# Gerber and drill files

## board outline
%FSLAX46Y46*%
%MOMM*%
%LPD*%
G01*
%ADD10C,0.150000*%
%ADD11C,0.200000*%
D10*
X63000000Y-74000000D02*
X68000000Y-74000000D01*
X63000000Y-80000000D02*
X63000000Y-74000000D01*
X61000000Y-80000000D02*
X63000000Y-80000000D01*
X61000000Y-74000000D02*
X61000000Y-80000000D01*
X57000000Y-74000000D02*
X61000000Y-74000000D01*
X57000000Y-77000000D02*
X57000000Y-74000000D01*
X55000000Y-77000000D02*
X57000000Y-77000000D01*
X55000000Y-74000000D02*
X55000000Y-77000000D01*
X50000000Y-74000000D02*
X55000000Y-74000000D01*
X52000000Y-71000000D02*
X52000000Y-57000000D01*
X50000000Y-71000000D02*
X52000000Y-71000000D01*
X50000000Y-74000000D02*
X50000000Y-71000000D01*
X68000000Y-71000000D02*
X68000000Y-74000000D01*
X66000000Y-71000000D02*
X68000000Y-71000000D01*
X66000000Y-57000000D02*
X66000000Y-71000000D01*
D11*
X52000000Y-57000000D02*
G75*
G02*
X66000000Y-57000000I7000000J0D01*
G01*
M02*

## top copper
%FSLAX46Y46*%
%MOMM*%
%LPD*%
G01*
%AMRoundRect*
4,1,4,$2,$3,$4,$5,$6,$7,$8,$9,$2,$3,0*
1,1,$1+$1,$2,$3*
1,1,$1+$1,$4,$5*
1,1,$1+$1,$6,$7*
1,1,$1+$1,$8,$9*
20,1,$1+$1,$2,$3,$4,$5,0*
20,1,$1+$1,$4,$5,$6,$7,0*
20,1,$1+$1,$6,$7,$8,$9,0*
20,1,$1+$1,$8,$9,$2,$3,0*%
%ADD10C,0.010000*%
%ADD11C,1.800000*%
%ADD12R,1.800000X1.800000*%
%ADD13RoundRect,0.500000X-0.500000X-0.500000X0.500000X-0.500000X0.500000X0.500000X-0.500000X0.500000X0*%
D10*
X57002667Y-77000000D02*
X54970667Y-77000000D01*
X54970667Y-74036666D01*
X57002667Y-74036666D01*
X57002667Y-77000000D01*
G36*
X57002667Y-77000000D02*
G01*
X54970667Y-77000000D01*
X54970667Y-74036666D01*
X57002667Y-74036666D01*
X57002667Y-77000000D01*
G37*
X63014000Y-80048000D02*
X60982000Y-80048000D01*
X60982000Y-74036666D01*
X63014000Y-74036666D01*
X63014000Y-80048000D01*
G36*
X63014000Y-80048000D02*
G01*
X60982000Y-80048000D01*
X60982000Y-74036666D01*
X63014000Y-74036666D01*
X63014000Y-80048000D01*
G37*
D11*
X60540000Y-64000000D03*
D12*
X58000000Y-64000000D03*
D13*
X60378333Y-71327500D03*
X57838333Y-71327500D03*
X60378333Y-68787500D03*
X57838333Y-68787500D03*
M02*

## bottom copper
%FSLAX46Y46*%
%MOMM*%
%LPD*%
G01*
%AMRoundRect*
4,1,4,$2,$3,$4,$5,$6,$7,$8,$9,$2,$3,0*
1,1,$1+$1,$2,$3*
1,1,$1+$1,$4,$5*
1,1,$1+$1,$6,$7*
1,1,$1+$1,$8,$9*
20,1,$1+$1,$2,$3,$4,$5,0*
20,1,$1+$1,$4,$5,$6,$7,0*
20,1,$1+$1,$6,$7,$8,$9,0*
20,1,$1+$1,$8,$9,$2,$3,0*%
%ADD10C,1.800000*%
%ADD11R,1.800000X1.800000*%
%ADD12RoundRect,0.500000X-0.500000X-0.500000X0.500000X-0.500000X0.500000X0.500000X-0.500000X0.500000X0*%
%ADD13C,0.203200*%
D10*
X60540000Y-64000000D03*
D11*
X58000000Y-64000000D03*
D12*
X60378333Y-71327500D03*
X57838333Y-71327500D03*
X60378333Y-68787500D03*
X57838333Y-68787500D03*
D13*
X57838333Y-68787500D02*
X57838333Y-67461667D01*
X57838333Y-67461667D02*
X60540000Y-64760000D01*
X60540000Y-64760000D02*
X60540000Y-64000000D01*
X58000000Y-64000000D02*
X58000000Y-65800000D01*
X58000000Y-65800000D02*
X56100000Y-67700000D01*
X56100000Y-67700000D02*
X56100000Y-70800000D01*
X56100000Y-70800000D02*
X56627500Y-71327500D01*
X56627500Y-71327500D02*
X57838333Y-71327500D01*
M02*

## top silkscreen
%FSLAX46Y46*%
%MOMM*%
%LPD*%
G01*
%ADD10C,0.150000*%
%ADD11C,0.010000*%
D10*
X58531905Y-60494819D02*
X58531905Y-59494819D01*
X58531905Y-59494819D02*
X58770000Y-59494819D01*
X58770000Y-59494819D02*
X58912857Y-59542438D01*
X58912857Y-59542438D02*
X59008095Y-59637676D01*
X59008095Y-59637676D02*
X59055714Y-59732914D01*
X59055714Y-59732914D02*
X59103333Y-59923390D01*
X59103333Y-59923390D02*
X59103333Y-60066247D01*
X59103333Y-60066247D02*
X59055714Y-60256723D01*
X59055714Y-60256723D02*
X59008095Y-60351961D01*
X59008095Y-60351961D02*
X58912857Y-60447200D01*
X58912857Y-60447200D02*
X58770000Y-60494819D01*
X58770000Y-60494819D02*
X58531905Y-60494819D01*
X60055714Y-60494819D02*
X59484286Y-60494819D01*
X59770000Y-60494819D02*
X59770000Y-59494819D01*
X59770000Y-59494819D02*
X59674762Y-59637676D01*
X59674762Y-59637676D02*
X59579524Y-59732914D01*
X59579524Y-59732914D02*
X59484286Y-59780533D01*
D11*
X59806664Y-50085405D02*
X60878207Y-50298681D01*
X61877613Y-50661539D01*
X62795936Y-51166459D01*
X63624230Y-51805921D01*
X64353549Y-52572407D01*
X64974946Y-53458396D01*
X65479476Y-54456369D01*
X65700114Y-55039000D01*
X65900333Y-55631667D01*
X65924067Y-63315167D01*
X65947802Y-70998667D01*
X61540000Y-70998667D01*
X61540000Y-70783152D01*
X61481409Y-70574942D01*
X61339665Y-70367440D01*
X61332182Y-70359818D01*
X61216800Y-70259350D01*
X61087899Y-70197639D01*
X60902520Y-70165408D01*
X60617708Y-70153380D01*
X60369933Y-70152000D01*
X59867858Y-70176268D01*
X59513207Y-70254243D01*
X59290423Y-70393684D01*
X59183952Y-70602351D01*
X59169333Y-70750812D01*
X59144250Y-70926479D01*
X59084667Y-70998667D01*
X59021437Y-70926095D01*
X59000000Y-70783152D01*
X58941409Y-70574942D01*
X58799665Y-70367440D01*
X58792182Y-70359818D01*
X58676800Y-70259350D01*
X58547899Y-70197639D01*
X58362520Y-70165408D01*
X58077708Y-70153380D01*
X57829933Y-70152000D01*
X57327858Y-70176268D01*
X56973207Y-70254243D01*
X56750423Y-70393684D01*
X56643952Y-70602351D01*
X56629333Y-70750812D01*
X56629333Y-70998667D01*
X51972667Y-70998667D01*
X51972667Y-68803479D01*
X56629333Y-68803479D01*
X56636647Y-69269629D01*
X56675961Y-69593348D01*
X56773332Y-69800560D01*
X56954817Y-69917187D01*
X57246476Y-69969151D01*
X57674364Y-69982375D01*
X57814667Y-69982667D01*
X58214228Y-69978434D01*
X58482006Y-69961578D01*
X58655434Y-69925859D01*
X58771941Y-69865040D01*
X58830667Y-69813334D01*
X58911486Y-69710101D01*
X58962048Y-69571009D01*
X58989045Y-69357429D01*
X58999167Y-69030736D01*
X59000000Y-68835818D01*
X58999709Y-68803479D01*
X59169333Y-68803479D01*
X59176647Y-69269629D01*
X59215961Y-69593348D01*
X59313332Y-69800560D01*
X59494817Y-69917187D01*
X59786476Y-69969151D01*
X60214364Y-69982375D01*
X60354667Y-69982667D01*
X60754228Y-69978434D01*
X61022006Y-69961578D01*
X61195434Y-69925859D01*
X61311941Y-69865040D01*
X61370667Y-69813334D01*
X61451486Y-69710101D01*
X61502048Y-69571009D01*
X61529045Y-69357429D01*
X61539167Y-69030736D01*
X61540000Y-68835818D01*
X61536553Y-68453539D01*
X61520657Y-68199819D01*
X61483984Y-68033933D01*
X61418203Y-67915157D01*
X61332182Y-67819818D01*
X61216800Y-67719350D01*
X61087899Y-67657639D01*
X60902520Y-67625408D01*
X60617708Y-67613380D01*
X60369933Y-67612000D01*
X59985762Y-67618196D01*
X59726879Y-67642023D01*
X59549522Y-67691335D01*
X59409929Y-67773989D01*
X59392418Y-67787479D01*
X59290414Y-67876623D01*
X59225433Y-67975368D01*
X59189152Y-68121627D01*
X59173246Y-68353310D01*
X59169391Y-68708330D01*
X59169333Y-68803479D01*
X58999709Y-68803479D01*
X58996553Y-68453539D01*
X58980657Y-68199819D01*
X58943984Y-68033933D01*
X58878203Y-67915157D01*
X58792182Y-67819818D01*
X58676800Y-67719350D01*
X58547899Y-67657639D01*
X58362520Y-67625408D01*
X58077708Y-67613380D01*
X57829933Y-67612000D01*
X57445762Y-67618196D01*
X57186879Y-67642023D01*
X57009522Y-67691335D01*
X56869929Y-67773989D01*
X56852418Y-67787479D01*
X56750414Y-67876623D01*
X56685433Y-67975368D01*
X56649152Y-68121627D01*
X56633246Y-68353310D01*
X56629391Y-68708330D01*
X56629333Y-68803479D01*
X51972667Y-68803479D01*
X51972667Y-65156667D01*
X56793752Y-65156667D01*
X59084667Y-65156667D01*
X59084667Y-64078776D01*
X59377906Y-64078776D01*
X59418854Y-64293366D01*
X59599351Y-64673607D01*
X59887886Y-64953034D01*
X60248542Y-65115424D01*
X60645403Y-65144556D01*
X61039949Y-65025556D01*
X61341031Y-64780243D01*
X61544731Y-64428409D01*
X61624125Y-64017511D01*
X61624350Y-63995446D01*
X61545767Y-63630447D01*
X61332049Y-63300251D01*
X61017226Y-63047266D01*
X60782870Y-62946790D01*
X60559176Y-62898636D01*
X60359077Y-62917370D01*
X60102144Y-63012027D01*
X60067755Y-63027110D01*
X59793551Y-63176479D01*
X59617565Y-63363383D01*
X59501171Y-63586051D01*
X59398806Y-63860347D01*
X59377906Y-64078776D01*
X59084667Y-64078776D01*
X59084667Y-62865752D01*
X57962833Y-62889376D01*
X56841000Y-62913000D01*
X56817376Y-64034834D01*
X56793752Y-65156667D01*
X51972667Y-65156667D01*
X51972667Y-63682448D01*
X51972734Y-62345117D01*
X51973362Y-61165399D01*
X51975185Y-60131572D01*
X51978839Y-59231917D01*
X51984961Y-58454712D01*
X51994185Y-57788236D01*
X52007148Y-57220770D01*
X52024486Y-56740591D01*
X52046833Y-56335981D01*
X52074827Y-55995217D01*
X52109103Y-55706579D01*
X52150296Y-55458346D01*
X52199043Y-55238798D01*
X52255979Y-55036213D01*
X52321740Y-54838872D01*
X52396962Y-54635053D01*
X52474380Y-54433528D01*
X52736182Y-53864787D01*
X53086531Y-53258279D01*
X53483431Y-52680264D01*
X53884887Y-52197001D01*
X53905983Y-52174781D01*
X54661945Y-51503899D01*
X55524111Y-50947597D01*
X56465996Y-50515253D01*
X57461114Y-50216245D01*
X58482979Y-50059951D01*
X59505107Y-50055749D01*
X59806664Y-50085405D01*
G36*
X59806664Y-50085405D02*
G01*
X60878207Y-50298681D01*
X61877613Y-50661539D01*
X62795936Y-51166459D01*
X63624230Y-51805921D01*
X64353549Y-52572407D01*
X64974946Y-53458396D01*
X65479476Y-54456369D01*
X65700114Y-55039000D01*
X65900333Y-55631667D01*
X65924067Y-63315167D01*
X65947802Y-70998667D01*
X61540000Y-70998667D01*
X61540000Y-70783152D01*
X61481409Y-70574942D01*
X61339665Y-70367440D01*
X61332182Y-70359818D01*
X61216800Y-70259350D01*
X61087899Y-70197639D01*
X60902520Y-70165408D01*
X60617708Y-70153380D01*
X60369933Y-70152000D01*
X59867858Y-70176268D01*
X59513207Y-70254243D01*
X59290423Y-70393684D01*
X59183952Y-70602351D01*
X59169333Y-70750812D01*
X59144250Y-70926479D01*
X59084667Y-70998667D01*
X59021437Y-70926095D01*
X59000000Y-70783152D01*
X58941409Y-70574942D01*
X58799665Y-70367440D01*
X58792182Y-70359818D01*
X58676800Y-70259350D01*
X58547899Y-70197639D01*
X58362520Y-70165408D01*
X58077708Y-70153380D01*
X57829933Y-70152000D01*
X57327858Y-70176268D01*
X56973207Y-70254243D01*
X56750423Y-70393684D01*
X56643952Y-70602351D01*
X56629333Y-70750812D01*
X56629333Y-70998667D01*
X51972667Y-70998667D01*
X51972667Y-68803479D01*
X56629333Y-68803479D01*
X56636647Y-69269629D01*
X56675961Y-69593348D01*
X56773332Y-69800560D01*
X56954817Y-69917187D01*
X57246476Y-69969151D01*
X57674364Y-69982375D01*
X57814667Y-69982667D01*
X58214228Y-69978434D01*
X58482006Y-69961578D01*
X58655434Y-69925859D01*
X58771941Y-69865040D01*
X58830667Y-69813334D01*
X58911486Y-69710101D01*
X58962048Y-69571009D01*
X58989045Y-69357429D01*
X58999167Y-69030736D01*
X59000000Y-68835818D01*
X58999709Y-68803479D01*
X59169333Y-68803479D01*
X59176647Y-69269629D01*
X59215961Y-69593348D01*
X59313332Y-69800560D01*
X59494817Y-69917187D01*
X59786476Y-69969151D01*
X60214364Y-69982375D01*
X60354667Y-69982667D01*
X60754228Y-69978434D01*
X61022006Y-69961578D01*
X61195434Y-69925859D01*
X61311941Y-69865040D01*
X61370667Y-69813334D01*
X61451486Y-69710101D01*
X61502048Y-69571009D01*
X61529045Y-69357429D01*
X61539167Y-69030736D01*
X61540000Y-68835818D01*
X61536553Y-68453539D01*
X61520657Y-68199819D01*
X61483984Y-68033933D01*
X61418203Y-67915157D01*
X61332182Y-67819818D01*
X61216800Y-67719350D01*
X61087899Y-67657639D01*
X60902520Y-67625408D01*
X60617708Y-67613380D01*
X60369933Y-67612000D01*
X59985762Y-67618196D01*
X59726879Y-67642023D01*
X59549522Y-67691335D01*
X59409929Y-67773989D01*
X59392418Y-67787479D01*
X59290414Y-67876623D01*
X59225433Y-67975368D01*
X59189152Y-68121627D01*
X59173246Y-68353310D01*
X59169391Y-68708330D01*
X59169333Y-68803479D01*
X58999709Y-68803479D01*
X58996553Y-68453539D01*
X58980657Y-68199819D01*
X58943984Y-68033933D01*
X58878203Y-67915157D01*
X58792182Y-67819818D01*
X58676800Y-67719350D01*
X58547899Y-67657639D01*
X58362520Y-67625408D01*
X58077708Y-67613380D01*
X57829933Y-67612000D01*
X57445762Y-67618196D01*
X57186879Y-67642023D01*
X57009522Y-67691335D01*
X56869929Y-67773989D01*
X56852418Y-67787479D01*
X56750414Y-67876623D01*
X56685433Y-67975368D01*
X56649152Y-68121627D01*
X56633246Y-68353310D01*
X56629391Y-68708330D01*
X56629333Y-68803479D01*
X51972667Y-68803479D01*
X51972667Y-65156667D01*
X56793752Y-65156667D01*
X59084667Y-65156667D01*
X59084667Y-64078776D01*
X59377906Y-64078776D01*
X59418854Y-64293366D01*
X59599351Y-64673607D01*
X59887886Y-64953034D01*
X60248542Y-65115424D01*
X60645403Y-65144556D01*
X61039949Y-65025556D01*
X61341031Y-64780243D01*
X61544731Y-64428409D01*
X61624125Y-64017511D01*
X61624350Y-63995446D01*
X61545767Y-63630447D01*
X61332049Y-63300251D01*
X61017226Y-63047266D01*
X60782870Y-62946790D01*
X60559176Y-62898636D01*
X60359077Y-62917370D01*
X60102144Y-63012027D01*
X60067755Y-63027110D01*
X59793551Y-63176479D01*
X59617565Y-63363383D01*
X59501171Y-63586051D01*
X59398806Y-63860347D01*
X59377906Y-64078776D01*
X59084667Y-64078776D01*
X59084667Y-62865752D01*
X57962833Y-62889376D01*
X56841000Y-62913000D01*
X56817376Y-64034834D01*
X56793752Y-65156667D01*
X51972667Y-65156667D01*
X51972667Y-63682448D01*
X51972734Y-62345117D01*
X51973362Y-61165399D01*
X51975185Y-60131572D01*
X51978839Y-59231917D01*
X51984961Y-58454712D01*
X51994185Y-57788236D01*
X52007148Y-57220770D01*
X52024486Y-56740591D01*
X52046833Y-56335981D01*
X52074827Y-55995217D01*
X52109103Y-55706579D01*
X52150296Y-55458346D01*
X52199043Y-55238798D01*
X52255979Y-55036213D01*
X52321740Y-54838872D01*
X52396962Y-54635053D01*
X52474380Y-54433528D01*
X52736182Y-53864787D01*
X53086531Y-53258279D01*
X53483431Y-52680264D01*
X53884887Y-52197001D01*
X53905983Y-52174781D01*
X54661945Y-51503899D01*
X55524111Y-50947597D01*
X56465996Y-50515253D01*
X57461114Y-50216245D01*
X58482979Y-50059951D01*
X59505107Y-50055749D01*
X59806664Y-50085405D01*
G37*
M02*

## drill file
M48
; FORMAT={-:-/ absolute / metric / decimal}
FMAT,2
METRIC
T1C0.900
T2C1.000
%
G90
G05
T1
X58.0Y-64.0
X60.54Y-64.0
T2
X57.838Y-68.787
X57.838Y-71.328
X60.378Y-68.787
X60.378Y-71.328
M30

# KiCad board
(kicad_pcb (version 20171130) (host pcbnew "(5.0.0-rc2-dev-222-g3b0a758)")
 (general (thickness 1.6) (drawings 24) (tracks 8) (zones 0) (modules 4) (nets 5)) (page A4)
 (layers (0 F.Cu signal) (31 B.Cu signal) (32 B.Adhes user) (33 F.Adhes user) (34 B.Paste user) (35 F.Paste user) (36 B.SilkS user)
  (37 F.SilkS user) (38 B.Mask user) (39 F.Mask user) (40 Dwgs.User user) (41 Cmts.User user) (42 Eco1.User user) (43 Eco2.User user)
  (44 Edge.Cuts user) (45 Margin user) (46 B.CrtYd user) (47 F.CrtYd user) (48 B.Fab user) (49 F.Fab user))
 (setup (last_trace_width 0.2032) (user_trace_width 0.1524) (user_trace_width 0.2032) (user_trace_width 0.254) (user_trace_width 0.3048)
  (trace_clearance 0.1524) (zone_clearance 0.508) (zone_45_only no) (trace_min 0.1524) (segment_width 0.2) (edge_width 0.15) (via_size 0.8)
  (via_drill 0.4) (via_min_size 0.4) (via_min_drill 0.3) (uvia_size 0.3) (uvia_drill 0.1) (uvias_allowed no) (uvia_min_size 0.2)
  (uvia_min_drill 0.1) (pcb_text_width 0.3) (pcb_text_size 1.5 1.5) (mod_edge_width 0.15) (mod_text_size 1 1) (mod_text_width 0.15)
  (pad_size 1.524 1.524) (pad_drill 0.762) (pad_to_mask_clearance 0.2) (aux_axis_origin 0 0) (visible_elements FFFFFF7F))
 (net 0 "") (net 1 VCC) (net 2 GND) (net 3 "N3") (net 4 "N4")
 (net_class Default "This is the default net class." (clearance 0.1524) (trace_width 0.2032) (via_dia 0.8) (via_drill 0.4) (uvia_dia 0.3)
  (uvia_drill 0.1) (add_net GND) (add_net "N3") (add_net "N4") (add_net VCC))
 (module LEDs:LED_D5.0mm (layer F.Cu) (at 58 64)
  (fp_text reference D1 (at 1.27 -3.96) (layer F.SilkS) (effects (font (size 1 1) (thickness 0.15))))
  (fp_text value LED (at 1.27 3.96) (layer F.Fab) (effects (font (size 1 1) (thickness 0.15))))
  (pad 2 thru_hole circle (at 2.54 0) (size 1.8 1.8) (drill 0.9) (layers *.Cu *.Mask) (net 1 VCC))
  (pad 1 thru_hole rect (at 0 0) (size 1.8 1.8) (drill 0.9) (layers *.Cu *.Mask) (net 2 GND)))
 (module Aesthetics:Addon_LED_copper (layer F.Cu) (at 58.95 77)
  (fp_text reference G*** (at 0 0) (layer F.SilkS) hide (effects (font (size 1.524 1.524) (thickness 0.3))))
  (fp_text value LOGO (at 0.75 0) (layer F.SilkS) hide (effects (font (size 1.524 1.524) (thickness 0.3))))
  (fp_poly
   (pts (xy -1.947333 0) (xy -3.979333 0) (xy -3.979333 -2.963334) (xy -1.947333 -2.963334) (xy -1.947333 0)) (layer F.Cu) (width 0.01))
  (fp_poly (pts (xy 4.064 3.048) (xy 2.032 3.048) (xy 2.032 -2.963334) (xy 4.064 -2.963334) (xy 4.064 3.048)) (layer F.Cu) (width 0.01)))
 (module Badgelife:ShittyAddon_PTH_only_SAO (layer F.Cu) (at 57.838333 68.7875)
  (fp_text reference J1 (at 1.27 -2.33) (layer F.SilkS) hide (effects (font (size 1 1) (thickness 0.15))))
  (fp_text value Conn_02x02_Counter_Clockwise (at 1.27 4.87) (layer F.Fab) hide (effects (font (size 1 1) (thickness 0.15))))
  (pad 3 thru_hole roundrect (at 2.54 2.54) (size 2 2) (drill 1) (layers *.Cu *.Mask) (roundrect_rratio 0.25) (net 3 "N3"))
  (pad 2 thru_hole roundrect (at 0 2.54) (size 2 2) (drill 1) (layers *.Cu *.Mask) (roundrect_rratio 0.25) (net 2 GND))
  (pad 4 thru_hole roundrect (at 2.54 0) (size 2 2) (drill 1) (layers *.Cu *.Mask) (roundrect_rratio 0.25) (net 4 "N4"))
  (pad 1 thru_hole roundrect (at 0 0) (size 2 2) (drill 1) (layers *.Cu *.Mask) (roundrect_rratio 0.25) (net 1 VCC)))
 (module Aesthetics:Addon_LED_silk (layer F.Cu) (at 59 60.5)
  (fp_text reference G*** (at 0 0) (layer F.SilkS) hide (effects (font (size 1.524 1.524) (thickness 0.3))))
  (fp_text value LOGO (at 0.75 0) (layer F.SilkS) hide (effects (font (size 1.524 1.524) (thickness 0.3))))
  (fp_poly
   (pts (xy 0.806664 -10.414595) (xy 1.878207 -10.201319) (xy 2.877613 -9.838461) (xy 3.795936 -9.333541) (xy 4.62423 -8.694079)
    (xy 5.353549 -7.927593) (xy 5.974946 -7.041604) (xy 6.479476 -6.043631) (xy 6.700114 -5.461) (xy 6.900333 -4.868333)
    (xy 6.924067 2.815167) (xy 6.947802 10.498667) (xy 2.54 10.498667) (xy 2.54 10.283152) (xy 2.481409 10.074942) (xy 2.339665 9.86744)
    (xy 2.332182 9.859818) (xy 2.2168 9.75935) (xy 2.087899 9.697639) (xy 1.90252 9.665408) (xy 1.617708 9.65338) (xy 1.369933 9.652)
    (xy 0.867858 9.676268) (xy 0.513207 9.754243) (xy 0.290423 9.893684) (xy 0.183952 10.102351) (xy 0.169333 10.250812)
    (xy 0.14425 10.426479) (xy 0.084667 10.498667) (xy 0.021437 10.426095) (xy 0 10.283152) (xy -0.058591 10.074942) (xy -0.200335 9.86744)
    (xy -0.207818 9.859818) (xy -0.3232 9.75935) (xy -0.452101 9.697639) (xy -0.63748 9.665408) (xy -0.922292 9.65338) (xy -1.170067 9.652)
    (xy -1.672142 9.676268) (xy -2.026793 9.754243) (xy -2.249577 9.893684) (xy -2.356048 10.102351) (xy -2.370667 10.250812)
    (xy -2.370667 10.498667) (xy -7.027333 10.498667) (xy -7.027333 8.303479) (xy -2.370667 8.303479) (xy -2.363353 8.769629)
    (xy -2.324039 9.093348) (xy -2.226668 9.30056) (xy -2.045183 9.417187) (xy -1.753524 9.469151) (xy -1.325636 9.482375)
    (xy -1.185333 9.482667) (xy -0.785772 9.478434) (xy -0.517994 9.461578) (xy -0.344566 9.425859) (xy -0.228059 9.36504)
    (xy -0.169333 9.313334) (xy -0.088514 9.210101) (xy -0.037952 9.071009) (xy -0.010955 8.857429) (xy -0.000833 8.530736) (xy 0 8.335818)
    (xy -0.000291 8.303479) (xy 0.169333 8.303479) (xy 0.176647 8.769629) (xy 0.215961 9.093348) (xy 0.313332 9.30056)
    (xy 0.494817 9.417187) (xy 0.786476 9.469151) (xy 1.214364 9.482375) (xy 1.354667 9.482667) (xy 1.754228 9.478434)
    (xy 2.022006 9.461578) (xy 2.195434 9.425859) (xy 2.311941 9.36504) (xy 2.370667 9.313334) (xy 2.451486 9.210101) (xy 2.502048 9.071009)
    (xy 2.529045 8.857429) (xy 2.539167 8.530736) (xy 2.54 8.335818) (xy 2.536553 7.953539) (xy 2.520657 7.699819) (xy 2.483984 7.533933)
    (xy 2.418203 7.415157) (xy 2.332182 7.319818) (xy 2.2168 7.21935) (xy 2.087899 7.157639) (xy 1.90252 7.125408) (xy 1.617708 7.11338)
    (xy 1.369933 7.112) (xy 0.985762 7.118196) (xy 0.726879 7.142023) (xy 0.549522 7.191335) (xy 0.409929 7.273989) (xy 0.392418 7.287479)
    (xy 0.290414 7.376623) (xy 0.225433 7.475368) (xy 0.189152 7.621627) (xy 0.173246 7.85331) (xy 0.169391 8.20833) (xy 0.169333 8.303479)
    (xy -0.000291 8.303479) (xy -0.003447 7.953539) (xy -0.019343 7.699819) (xy -0.056016 7.533933) (xy -0.121797 7.415157)
    (xy -0.207818 7.319818) (xy -0.3232 7.21935) (xy -0.452101 7.157639) (xy -0.63748 7.125408) (xy -0.922292 7.11338) (xy -1.170067 7.112)
    (xy -1.554238 7.118196) (xy -1.813121 7.142023) (xy -1.990478 7.191335) (xy -2.130071 7.273989) (xy -2.147582 7.287479)
    (xy -2.249586 7.376623) (xy -2.314567 7.475368) (xy -2.350848 7.621627) (xy -2.366754 7.85331) (xy -2.370609 8.20833)
    (xy -2.370667 8.303479) (xy -7.027333 8.303479) (xy -7.027333 4.656667) (xy -2.206248 4.656667) (xy 0.084667 4.656667)
    (xy 0.084667 3.578776) (xy 0.377906 3.578776) (xy 0.418854 3.793366) (xy 0.599351 4.173607) (xy 0.887886 4.453034)
    (xy 1.248542 4.615424) (xy 1.645403 4.644556) (xy 2.039949 4.525556) (xy 2.341031 4.280243) (xy 2.544731 3.928409)
    (xy 2.624125 3.517511) (xy 2.62435 3.495446) (xy 2.545767 3.130447) (xy 2.332049 2.800251) (xy 2.017226 2.547266) (xy 1.78287 2.44679)
    (xy 1.559176 2.398636) (xy 1.359077 2.41737) (xy 1.102144 2.512027) (xy 1.067755 2.52711) (xy 0.793551 2.676479) (xy 0.617565 2.863383)
    (xy 0.501171 3.086051) (xy 0.398806 3.360347) (xy 0.377906 3.578776) (xy 0.084667 3.578776) (xy 0.084667 2.365752)
    (xy -1.037167 2.389376) (xy -2.159 2.413) (xy -2.182624 3.534834) (xy -2.206248 4.656667) (xy -7.027333 4.656667)
    (xy -7.027333 3.182448) (xy -7.027266 1.845117) (xy -7.026638 0.665399) (xy -7.024815 -0.368428) (xy -7.021161 -1.268083)
    (xy -7.015039 -2.045288) (xy -7.005815 -2.711764) (xy -6.992852 -3.27923) (xy -6.975514 -3.759409) (xy -6.953167 -4.164019)
    (xy -6.925173 -4.504783) (xy -6.890897 -4.793421) (xy -6.849704 -5.041654) (xy -6.800957 -5.261202) (xy -6.744021 -5.463787)
    (xy -6.67826 -5.661128) (xy -6.603038 -5.864947) (xy -6.52562 -6.066472) (xy -6.263818 -6.635213) (xy -5.913469 -7.241721)
    (xy -5.516569 -7.819736) (xy -5.115113 -8.302999) (xy -5.094017 -8.325219) (xy -4.338055 -8.996101) (xy -3.475889 -9.552403)
    (xy -2.534004 -9.984747) (xy -1.538886 -10.283755) (xy -0.517021 -10.440049) (xy 0.505107 -10.444251) (xy 0.806664 -10.414595))
   (layer F.SilkS) (width 0.01)))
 (gr_line (start 63 74) (end 68 74) (layer Edge.Cuts) (width 0.15))
 (gr_line (start 63 80) (end 63 74) (layer Edge.Cuts) (width 0.15))
 (gr_line (start 61 80) (end 63 80) (layer Edge.Cuts) (width 0.15))
 (gr_line (start 61 74) (end 61 80) (layer Edge.Cuts) (width 0.15))
 (gr_line (start 57 74) (end 61 74) (layer Edge.Cuts) (width 0.15))
 (gr_line (start 57 77) (end 57 74) (layer Edge.Cuts) (width 0.15))
 (gr_line (start 55 77) (end 57 77) (layer Edge.Cuts) (width 0.15))
 (gr_line (start 55 74) (end 55 77) (layer Edge.Cuts) (width 0.15))
 (gr_line (start 50 74) (end 55 74) (layer Edge.Cuts) (width 0.15))
 (gr_line (start 52 71) (end 52 57) (layer Edge.Cuts) (width 0.15))
 (gr_line (start 50 71) (end 52 71) (layer Edge.Cuts) (width 0.15))
 (gr_line (start 50 74) (end 50 71) (layer Edge.Cuts) (width 0.15))
 (gr_line (start 68 71) (end 68 74) (layer Edge.Cuts) (width 0.15))
 (gr_line (start 66 71) (end 68 71) (layer Edge.Cuts) (width 0.15))
 (gr_line (start 66 57) (end 66 71) (layer Edge.Cuts) (width 0.15))
 (gr_arc (start 59 57) (end 66 57) (angle -180) (layer Edge.Cuts) (width 0.2))
 (segment (start 57.838333 68.7875) (end 57.838333 67.461667) (width 0.2032) (layer B.Cu) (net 1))
 (segment (start 57.838333 67.461667) (end 60.54 64.76) (width 0.2032) (layer B.Cu) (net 1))
 (segment (start 60.54 64.76) (end 60.54 64) (width 0.2032) (layer B.Cu) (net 1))
 (segment (start 58 64) (end 58 65.8) (width 0.2032) (layer B.Cu) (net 2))
 (segment (start 58 65.8) (end 56.1 67.7) (width 0.2032) (layer B.Cu) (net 2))
 (segment (start 56.1 67.7) (end 56.1 70.8) (width 0.2032) (layer B.Cu) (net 2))
 (segment (start 56.1 70.8) (end 56.6275 71.3275) (width 0.2032) (layer B.Cu) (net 2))
 (segment (start 56.6275 71.3275) (end 57.838333 71.3275) (width 0.2032) (layer B.Cu) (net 2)))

